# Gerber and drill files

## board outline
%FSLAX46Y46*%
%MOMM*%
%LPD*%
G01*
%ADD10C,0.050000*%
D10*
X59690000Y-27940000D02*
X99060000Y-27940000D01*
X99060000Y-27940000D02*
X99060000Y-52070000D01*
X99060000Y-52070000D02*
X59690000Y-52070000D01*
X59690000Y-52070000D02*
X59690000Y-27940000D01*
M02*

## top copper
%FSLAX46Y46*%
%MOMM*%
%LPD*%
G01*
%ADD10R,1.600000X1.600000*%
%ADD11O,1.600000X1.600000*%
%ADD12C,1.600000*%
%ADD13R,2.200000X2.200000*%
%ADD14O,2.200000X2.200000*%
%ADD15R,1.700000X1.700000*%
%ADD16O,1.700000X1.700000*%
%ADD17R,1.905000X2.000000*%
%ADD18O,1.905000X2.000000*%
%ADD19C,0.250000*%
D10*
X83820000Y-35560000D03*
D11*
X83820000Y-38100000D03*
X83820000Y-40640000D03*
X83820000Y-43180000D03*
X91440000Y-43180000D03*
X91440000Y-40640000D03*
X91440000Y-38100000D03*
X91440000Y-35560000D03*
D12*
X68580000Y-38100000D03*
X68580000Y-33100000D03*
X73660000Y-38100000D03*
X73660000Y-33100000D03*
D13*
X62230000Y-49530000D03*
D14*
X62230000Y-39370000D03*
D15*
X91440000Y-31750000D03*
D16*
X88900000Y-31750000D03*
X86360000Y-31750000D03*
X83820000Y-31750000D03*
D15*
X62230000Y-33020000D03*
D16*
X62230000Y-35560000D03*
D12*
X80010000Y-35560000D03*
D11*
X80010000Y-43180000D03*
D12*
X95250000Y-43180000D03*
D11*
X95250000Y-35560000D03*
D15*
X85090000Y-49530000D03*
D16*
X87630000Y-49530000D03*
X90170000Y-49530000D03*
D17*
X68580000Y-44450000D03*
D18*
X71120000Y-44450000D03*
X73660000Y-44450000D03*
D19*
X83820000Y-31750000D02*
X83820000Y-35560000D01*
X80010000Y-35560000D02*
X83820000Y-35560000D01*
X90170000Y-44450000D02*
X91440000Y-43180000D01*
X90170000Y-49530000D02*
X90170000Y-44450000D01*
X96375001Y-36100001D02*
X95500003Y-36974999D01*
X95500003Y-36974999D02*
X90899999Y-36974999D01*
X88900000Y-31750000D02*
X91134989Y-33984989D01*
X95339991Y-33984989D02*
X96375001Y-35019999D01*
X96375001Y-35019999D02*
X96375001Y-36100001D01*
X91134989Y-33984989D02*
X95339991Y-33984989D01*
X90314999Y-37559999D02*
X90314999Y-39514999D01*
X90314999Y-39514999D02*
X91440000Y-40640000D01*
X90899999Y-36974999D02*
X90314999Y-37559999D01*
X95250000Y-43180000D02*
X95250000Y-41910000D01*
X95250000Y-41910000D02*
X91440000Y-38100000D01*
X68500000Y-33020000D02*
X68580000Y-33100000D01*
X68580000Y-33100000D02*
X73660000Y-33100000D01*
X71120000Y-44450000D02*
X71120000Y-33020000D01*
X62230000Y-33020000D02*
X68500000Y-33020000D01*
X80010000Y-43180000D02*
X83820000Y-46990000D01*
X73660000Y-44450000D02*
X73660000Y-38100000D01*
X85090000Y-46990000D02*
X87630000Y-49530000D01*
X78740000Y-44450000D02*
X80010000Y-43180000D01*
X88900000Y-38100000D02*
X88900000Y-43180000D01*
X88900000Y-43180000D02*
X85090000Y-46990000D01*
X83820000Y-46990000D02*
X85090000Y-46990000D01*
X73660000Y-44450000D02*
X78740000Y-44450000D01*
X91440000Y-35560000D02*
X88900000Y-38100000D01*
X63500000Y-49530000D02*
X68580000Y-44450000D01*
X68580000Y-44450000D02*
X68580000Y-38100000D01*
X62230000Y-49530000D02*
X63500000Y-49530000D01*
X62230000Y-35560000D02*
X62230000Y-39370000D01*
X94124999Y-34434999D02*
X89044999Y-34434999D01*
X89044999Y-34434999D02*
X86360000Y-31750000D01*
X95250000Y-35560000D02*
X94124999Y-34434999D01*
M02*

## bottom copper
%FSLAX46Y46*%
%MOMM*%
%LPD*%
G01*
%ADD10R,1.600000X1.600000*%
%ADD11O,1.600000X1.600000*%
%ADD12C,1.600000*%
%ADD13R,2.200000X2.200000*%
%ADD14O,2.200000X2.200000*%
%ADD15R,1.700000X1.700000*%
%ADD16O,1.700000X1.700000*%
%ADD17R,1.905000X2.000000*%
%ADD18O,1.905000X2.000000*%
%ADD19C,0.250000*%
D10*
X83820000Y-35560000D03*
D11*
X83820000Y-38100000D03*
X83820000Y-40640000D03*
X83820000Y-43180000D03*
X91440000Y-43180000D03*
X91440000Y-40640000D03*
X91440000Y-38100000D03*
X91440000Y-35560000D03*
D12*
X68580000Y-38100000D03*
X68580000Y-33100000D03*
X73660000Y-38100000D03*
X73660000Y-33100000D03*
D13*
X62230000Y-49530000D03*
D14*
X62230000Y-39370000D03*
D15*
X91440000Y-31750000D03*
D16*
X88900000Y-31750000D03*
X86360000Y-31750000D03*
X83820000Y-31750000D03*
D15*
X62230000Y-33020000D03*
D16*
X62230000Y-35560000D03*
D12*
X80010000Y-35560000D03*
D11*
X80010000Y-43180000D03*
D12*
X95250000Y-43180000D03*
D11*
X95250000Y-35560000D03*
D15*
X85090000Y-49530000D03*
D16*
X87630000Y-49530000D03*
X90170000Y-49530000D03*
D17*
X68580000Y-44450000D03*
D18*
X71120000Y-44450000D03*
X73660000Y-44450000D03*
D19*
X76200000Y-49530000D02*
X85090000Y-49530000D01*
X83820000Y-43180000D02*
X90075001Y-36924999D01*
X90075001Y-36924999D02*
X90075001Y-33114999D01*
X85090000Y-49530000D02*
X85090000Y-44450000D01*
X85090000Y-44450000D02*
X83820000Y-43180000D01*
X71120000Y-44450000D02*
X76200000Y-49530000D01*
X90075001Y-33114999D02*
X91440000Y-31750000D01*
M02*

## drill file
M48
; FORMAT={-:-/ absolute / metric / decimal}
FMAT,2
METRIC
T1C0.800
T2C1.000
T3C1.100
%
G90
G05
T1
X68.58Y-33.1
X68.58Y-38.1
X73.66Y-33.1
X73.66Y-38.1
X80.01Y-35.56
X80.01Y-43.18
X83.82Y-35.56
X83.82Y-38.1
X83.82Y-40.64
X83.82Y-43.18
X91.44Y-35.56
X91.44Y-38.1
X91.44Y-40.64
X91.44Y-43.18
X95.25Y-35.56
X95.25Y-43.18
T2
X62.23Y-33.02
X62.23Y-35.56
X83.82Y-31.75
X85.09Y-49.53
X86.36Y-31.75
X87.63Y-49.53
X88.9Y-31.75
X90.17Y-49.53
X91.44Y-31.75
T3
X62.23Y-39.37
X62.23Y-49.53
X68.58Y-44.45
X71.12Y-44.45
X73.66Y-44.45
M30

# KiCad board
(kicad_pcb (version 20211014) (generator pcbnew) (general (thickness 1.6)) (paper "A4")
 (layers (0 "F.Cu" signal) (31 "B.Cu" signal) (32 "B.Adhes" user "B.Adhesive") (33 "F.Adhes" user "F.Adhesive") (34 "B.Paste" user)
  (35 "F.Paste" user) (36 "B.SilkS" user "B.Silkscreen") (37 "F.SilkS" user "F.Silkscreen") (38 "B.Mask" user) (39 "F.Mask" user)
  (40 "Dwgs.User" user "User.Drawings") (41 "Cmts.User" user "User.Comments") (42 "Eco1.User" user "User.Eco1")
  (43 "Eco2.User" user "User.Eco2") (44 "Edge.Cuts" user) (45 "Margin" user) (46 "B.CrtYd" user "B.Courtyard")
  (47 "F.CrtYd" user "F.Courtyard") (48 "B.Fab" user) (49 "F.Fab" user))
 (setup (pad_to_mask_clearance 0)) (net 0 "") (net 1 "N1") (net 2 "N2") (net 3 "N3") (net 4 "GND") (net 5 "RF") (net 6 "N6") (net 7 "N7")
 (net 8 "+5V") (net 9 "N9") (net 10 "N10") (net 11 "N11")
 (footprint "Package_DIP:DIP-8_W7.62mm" (layer "F.Cu") (at 83.82 35.56)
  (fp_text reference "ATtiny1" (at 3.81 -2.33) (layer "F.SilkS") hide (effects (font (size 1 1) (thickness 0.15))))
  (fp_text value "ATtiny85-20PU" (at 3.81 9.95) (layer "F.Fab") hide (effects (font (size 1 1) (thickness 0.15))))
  (pad "1" thru_hole rect locked (at 0 0) (size 1.6 1.6) (drill 0.8) (layers *.Cu *.Mask) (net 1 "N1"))
  (pad "2" thru_hole oval locked (at 0 2.54) (size 1.6 1.6) (drill 0.8) (layers *.Cu *.Mask) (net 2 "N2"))
  (pad "3" thru_hole oval locked (at 0 5.08) (size 1.6 1.6) (drill 0.8) (layers *.Cu *.Mask) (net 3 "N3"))
  (pad "4" thru_hole oval locked (at 0 7.62) (size 1.6 1.6) (drill 0.8) (layers *.Cu *.Mask) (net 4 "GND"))
  (pad "5" thru_hole oval locked (at 7.62 7.62) (size 1.6 1.6) (drill 0.8) (layers *.Cu *.Mask) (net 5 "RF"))
  (pad "6" thru_hole oval locked (at 7.62 5.08) (size 1.6 1.6) (drill 0.8) (layers *.Cu *.Mask) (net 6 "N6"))
  (pad "7" thru_hole oval locked (at 7.62 2.54) (size 1.6 1.6) (drill 0.8) (layers *.Cu *.Mask) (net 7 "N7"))
  (pad "8" thru_hole oval locked (at 7.62 0) (size 1.6 1.6) (drill 0.8) (layers *.Cu *.Mask) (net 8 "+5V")))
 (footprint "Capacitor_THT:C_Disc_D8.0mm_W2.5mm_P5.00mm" (layer "F.Cu") (at 68.58 38.1 90)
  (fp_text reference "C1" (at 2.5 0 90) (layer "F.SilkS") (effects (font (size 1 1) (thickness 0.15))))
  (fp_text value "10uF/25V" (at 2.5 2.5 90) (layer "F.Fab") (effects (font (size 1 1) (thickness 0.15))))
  (pad "1" thru_hole circle locked (at 0 0 90) (size 1.6 1.6) (drill 0.8) (layers *.Cu *.Mask) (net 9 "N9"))
  (pad "2" thru_hole circle locked (at 5 0 90) (size 1.6 1.6) (drill 0.8) (layers *.Cu *.Mask) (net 4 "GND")))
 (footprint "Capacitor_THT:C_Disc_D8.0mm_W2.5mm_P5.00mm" (layer "F.Cu") (at 73.66 38.1 90)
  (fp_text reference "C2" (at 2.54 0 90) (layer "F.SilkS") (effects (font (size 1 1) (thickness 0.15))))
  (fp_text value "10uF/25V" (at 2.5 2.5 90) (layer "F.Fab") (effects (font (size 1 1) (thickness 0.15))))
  (pad "1" thru_hole circle locked (at 0 0 90) (size 1.6 1.6) (drill 0.8) (layers *.Cu *.Mask) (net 8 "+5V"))
  (pad "2" thru_hole circle locked (at 5 0 90) (size 1.6 1.6) (drill 0.8) (layers *.Cu *.Mask) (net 4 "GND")))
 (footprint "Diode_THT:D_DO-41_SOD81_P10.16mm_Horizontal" (layer "F.Cu") (at 62.23 49.53 90)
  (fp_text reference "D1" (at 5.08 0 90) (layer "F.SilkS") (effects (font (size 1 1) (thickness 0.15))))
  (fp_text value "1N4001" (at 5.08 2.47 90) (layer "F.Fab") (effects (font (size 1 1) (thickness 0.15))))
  (pad "1" thru_hole rect locked (at 0 0 90) (size 2.2 2.2) (drill 1.1) (layers *.Cu *.Mask) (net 9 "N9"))
  (pad "2" thru_hole oval locked (at 10.16 0 90) (size 2.2 2.2) (drill 1.1) (layers *.Cu *.Mask) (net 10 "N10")))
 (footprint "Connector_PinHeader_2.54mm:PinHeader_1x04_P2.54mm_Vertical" (layer "F.Cu") (at 91.44 31.75 -90)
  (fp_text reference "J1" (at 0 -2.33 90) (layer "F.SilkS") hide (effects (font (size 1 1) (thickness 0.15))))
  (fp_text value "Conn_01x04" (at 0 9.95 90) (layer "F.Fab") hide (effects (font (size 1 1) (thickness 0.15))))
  (pad "1" thru_hole rect locked (at 0 0 270) (size 1.7 1.7) (drill 1) (layers *.Cu *.Mask) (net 4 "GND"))
  (pad "2" thru_hole oval locked (at 0 2.54 270) (size 1.7 1.7) (drill 1) (layers *.Cu *.Mask) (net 6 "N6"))
  (pad "3" thru_hole oval locked (at 0 5.08 270) (size 1.7 1.7) (drill 1) (layers *.Cu *.Mask) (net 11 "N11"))
  (pad "4" thru_hole oval locked (at 0 7.62 270) (size 1.7 1.7) (drill 1) (layers *.Cu *.Mask) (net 1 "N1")))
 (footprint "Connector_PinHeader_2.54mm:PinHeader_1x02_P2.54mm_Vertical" (layer "F.Cu") (at 62.23 33.02)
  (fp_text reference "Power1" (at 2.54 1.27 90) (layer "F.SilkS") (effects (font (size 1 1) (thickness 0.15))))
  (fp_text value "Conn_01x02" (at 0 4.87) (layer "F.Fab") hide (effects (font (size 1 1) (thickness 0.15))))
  (pad "1" thru_hole rect locked (at 0 0) (size 1.7 1.7) (drill 1) (layers *.Cu *.Mask) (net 4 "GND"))
  (pad "2" thru_hole oval locked (at 0 2.54) (size 1.7 1.7) (drill 1) (layers *.Cu *.Mask) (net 10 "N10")))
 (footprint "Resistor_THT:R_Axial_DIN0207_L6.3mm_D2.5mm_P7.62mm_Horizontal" (layer "F.Cu") (at 80.01 35.56 -90)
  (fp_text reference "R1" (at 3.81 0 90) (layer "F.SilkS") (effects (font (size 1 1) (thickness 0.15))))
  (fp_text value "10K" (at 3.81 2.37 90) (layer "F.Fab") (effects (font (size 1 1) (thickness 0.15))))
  (pad "1" thru_hole circle locked (at 0 0 270) (size 1.6 1.6) (drill 0.8) (layers *.Cu *.Mask) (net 1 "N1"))
  (pad "2" thru_hole oval locked (at 7.62 0 270) (size 1.6 1.6) (drill 0.8) (layers *.Cu *.Mask) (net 8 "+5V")))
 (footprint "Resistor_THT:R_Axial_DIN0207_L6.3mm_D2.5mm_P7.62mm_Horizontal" (layer "F.Cu") (at 95.25 43.18 90)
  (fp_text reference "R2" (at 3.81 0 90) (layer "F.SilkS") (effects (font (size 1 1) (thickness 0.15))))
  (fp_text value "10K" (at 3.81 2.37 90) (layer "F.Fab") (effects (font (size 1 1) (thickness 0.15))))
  (pad "1" thru_hole circle locked (at 0 0 90) (size 1.6 1.6) (drill 0.8) (layers *.Cu *.Mask) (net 7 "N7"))
  (pad "2" thru_hole oval locked (at 7.62 0 90) (size 1.6 1.6) (drill 0.8) (layers *.Cu *.Mask) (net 11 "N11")))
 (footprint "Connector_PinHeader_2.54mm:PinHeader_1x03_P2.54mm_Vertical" (layer "F.Cu") (at 85.09 49.53 90)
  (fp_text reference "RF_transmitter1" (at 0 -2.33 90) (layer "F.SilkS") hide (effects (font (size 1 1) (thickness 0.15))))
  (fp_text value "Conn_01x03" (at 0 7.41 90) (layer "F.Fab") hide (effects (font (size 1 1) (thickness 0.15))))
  (pad "1" thru_hole rect locked (at 0 0 90) (size 1.7 1.7) (drill 1) (layers *.Cu *.Mask) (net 4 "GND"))
  (pad "2" thru_hole oval locked (at 0 2.54 90) (size 1.7 1.7) (drill 1) (layers *.Cu *.Mask) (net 8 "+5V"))
  (pad "3" thru_hole oval locked (at 0 5.08 90) (size 1.7 1.7) (drill 1) (layers *.Cu *.Mask) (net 5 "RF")))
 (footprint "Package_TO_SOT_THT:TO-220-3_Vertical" (layer "F.Cu") (at 68.58 44.45)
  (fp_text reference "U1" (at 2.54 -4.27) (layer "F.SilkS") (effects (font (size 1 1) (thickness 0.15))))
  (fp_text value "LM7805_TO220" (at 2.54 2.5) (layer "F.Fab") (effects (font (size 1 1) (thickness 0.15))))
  (pad "1" thru_hole rect locked (at 0 0) (size 1.905 2) (drill 1.1) (layers *.Cu *.Mask) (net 9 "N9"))
  (pad "2" thru_hole oval locked (at 2.54 0) (size 1.905 2) (drill 1.1) (layers *.Cu *.Mask) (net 4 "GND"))
  (pad "3" thru_hole oval locked (at 5.08 0) (size 1.905 2) (drill 1.1) (layers *.Cu *.Mask) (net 8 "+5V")))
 (gr_line (start 59.69 27.94) (end 99.06 27.94) (layer "Edge.Cuts") (width 0.05))
 (gr_line (start 99.06 27.94) (end 99.06 52.07) (layer "Edge.Cuts") (width 0.05))
 (gr_line (start 99.06 52.07) (end 59.69 52.07) (layer "Edge.Cuts") (width 0.05))
 (gr_line (start 59.69 52.07) (end 59.69 27.94) (layer "Edge.Cuts") (width 0.05))
 (segment (start 83.82 31.75) (end 83.82 35.56) (width 0.25) (layer "F.Cu") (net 1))
 (segment (start 80.01 35.56) (end 83.82 35.56) (width 0.25) (layer "F.Cu") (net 1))
 (segment (start 90.17 44.45) (end 91.44 43.18) (width 0.25) (layer "F.Cu") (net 5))
 (segment (start 90.17 49.53) (end 90.17 44.45) (width 0.25) (layer "F.Cu") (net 5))
 (segment (start 96.375001 36.100001) (end 95.500003 36.974999) (width 0.25) (layer "F.Cu") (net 6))
 (segment (start 95.500003 36.974999) (end 90.899999 36.974999) (width 0.25) (layer "F.Cu") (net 6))
 (segment (start 88.9 31.75) (end 91.134989 33.984989) (width 0.25) (layer "F.Cu") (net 6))
 (segment (start 95.339991 33.984989) (end 96.375001 35.019999) (width 0.25) (layer "F.Cu") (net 6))
 (segment (start 96.375001 35.019999) (end 96.375001 36.100001) (width 0.25) (layer "F.Cu") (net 6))
 (segment (start 91.134989 33.984989) (end 95.339991 33.984989) (width 0.25) (layer "F.Cu") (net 6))
 (segment (start 90.314999 37.559999) (end 90.314999 39.514999) (width 0.25) (layer "F.Cu") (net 6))
 (segment (start 90.314999 39.514999) (end 91.44 40.64) (width 0.25) (layer "F.Cu") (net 6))
 (segment (start 90.899999 36.974999) (end 90.314999 37.559999) (width 0.25) (layer "F.Cu") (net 6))
 (segment (start 95.25 43.18) (end 95.25 41.91) (width 0.25) (layer "F.Cu") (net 7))
 (segment (start 95.25 41.91) (end 91.44 38.1) (width 0.25) (layer "F.Cu") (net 7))
 (segment (start 68.5 33.02) (end 68.58 33.1) (width 0.25) (layer "F.Cu") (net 4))
 (segment (start 68.58 33.1) (end 73.66 33.1) (width 0.25) (layer "F.Cu") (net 4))
 (segment (start 71.12 44.45) (end 71.12 33.02) (width 0.25) (layer "F.Cu") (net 4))
 (segment (start 62.23 33.02) (end 68.5 33.02) (width 0.25) (layer "F.Cu") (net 4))
 (segment (start 76.2 49.53) (end 85.09 49.53) (width 0.25) (layer "B.Cu") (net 4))
 (segment (start 83.82 43.18) (end 90.075001 36.924999) (width 0.25) (layer "B.Cu") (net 4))
 (segment (start 90.075001 36.924999) (end 90.075001 33.114999) (width 0.25) (layer "B.Cu") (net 4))
 (segment (start 85.09 49.53) (end 85.09 44.45) (width 0.25) (layer "B.Cu") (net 4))
 (segment (start 85.09 44.45) (end 83.82 43.18) (width 0.25) (layer "B.Cu") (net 4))
 (segment (start 71.12 44.45) (end 76.2 49.53) (width 0.25) (layer "B.Cu") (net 4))
 (segment (start 90.075001 33.114999) (end 91.44 31.75) (width 0.25) (layer "B.Cu") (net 4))
 (segment (start 80.01 43.18) (end 83.82 46.99) (width 0.25) (layer "F.Cu") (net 8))
 (segment (start 73.66 44.45) (end 73.66 38.1) (width 0.25) (layer "F.Cu") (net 8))
 (segment (start 85.09 46.99) (end 87.63 49.53) (width 0.25) (layer "F.Cu") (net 8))
 (segment (start 78.74 44.45) (end 80.01 43.18) (width 0.25) (layer "F.Cu") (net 8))
 (segment (start 88.9 38.1) (end 88.9 43.18) (width 0.25) (layer "F.Cu") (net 8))
 (segment (start 88.9 43.18) (end 85.09 46.99) (width 0.25) (layer "F.Cu") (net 8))
 (segment (start 83.82 46.99) (end 85.09 46.99) (width 0.25) (layer "F.Cu") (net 8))
 (segment (start 73.66 44.45) (end 78.74 44.45) (width 0.25) (layer "F.Cu") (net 8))
 (segment (start 91.44 35.56) (end 88.9 38.1) (width 0.25) (layer "F.Cu") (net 8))
 (segment (start 63.5 49.53) (end 68.58 44.45) (width 0.25) (layer "F.Cu") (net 9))
 (segment (start 68.58 44.45) (end 68.58 38.1) (width 0.25) (layer "F.Cu") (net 9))
 (segment (start 62.23 49.53) (end 63.5 49.53) (width 0.25) (layer "F.Cu") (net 9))
 (segment (start 62.23 35.56) (end 62.23 39.37) (width 0.25) (layer "F.Cu") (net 10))
 (segment (start 94.124999 34.434999) (end 89.044999 34.434999) (width 0.25) (layer "F.Cu") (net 11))
 (segment (start 89.044999 34.434999) (end 86.36 31.75) (width 0.25) (layer "F.Cu") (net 11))
 (segment (start 95.25 35.56) (end 94.124999 34.434999) (width 0.25) (layer "F.Cu") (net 11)))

